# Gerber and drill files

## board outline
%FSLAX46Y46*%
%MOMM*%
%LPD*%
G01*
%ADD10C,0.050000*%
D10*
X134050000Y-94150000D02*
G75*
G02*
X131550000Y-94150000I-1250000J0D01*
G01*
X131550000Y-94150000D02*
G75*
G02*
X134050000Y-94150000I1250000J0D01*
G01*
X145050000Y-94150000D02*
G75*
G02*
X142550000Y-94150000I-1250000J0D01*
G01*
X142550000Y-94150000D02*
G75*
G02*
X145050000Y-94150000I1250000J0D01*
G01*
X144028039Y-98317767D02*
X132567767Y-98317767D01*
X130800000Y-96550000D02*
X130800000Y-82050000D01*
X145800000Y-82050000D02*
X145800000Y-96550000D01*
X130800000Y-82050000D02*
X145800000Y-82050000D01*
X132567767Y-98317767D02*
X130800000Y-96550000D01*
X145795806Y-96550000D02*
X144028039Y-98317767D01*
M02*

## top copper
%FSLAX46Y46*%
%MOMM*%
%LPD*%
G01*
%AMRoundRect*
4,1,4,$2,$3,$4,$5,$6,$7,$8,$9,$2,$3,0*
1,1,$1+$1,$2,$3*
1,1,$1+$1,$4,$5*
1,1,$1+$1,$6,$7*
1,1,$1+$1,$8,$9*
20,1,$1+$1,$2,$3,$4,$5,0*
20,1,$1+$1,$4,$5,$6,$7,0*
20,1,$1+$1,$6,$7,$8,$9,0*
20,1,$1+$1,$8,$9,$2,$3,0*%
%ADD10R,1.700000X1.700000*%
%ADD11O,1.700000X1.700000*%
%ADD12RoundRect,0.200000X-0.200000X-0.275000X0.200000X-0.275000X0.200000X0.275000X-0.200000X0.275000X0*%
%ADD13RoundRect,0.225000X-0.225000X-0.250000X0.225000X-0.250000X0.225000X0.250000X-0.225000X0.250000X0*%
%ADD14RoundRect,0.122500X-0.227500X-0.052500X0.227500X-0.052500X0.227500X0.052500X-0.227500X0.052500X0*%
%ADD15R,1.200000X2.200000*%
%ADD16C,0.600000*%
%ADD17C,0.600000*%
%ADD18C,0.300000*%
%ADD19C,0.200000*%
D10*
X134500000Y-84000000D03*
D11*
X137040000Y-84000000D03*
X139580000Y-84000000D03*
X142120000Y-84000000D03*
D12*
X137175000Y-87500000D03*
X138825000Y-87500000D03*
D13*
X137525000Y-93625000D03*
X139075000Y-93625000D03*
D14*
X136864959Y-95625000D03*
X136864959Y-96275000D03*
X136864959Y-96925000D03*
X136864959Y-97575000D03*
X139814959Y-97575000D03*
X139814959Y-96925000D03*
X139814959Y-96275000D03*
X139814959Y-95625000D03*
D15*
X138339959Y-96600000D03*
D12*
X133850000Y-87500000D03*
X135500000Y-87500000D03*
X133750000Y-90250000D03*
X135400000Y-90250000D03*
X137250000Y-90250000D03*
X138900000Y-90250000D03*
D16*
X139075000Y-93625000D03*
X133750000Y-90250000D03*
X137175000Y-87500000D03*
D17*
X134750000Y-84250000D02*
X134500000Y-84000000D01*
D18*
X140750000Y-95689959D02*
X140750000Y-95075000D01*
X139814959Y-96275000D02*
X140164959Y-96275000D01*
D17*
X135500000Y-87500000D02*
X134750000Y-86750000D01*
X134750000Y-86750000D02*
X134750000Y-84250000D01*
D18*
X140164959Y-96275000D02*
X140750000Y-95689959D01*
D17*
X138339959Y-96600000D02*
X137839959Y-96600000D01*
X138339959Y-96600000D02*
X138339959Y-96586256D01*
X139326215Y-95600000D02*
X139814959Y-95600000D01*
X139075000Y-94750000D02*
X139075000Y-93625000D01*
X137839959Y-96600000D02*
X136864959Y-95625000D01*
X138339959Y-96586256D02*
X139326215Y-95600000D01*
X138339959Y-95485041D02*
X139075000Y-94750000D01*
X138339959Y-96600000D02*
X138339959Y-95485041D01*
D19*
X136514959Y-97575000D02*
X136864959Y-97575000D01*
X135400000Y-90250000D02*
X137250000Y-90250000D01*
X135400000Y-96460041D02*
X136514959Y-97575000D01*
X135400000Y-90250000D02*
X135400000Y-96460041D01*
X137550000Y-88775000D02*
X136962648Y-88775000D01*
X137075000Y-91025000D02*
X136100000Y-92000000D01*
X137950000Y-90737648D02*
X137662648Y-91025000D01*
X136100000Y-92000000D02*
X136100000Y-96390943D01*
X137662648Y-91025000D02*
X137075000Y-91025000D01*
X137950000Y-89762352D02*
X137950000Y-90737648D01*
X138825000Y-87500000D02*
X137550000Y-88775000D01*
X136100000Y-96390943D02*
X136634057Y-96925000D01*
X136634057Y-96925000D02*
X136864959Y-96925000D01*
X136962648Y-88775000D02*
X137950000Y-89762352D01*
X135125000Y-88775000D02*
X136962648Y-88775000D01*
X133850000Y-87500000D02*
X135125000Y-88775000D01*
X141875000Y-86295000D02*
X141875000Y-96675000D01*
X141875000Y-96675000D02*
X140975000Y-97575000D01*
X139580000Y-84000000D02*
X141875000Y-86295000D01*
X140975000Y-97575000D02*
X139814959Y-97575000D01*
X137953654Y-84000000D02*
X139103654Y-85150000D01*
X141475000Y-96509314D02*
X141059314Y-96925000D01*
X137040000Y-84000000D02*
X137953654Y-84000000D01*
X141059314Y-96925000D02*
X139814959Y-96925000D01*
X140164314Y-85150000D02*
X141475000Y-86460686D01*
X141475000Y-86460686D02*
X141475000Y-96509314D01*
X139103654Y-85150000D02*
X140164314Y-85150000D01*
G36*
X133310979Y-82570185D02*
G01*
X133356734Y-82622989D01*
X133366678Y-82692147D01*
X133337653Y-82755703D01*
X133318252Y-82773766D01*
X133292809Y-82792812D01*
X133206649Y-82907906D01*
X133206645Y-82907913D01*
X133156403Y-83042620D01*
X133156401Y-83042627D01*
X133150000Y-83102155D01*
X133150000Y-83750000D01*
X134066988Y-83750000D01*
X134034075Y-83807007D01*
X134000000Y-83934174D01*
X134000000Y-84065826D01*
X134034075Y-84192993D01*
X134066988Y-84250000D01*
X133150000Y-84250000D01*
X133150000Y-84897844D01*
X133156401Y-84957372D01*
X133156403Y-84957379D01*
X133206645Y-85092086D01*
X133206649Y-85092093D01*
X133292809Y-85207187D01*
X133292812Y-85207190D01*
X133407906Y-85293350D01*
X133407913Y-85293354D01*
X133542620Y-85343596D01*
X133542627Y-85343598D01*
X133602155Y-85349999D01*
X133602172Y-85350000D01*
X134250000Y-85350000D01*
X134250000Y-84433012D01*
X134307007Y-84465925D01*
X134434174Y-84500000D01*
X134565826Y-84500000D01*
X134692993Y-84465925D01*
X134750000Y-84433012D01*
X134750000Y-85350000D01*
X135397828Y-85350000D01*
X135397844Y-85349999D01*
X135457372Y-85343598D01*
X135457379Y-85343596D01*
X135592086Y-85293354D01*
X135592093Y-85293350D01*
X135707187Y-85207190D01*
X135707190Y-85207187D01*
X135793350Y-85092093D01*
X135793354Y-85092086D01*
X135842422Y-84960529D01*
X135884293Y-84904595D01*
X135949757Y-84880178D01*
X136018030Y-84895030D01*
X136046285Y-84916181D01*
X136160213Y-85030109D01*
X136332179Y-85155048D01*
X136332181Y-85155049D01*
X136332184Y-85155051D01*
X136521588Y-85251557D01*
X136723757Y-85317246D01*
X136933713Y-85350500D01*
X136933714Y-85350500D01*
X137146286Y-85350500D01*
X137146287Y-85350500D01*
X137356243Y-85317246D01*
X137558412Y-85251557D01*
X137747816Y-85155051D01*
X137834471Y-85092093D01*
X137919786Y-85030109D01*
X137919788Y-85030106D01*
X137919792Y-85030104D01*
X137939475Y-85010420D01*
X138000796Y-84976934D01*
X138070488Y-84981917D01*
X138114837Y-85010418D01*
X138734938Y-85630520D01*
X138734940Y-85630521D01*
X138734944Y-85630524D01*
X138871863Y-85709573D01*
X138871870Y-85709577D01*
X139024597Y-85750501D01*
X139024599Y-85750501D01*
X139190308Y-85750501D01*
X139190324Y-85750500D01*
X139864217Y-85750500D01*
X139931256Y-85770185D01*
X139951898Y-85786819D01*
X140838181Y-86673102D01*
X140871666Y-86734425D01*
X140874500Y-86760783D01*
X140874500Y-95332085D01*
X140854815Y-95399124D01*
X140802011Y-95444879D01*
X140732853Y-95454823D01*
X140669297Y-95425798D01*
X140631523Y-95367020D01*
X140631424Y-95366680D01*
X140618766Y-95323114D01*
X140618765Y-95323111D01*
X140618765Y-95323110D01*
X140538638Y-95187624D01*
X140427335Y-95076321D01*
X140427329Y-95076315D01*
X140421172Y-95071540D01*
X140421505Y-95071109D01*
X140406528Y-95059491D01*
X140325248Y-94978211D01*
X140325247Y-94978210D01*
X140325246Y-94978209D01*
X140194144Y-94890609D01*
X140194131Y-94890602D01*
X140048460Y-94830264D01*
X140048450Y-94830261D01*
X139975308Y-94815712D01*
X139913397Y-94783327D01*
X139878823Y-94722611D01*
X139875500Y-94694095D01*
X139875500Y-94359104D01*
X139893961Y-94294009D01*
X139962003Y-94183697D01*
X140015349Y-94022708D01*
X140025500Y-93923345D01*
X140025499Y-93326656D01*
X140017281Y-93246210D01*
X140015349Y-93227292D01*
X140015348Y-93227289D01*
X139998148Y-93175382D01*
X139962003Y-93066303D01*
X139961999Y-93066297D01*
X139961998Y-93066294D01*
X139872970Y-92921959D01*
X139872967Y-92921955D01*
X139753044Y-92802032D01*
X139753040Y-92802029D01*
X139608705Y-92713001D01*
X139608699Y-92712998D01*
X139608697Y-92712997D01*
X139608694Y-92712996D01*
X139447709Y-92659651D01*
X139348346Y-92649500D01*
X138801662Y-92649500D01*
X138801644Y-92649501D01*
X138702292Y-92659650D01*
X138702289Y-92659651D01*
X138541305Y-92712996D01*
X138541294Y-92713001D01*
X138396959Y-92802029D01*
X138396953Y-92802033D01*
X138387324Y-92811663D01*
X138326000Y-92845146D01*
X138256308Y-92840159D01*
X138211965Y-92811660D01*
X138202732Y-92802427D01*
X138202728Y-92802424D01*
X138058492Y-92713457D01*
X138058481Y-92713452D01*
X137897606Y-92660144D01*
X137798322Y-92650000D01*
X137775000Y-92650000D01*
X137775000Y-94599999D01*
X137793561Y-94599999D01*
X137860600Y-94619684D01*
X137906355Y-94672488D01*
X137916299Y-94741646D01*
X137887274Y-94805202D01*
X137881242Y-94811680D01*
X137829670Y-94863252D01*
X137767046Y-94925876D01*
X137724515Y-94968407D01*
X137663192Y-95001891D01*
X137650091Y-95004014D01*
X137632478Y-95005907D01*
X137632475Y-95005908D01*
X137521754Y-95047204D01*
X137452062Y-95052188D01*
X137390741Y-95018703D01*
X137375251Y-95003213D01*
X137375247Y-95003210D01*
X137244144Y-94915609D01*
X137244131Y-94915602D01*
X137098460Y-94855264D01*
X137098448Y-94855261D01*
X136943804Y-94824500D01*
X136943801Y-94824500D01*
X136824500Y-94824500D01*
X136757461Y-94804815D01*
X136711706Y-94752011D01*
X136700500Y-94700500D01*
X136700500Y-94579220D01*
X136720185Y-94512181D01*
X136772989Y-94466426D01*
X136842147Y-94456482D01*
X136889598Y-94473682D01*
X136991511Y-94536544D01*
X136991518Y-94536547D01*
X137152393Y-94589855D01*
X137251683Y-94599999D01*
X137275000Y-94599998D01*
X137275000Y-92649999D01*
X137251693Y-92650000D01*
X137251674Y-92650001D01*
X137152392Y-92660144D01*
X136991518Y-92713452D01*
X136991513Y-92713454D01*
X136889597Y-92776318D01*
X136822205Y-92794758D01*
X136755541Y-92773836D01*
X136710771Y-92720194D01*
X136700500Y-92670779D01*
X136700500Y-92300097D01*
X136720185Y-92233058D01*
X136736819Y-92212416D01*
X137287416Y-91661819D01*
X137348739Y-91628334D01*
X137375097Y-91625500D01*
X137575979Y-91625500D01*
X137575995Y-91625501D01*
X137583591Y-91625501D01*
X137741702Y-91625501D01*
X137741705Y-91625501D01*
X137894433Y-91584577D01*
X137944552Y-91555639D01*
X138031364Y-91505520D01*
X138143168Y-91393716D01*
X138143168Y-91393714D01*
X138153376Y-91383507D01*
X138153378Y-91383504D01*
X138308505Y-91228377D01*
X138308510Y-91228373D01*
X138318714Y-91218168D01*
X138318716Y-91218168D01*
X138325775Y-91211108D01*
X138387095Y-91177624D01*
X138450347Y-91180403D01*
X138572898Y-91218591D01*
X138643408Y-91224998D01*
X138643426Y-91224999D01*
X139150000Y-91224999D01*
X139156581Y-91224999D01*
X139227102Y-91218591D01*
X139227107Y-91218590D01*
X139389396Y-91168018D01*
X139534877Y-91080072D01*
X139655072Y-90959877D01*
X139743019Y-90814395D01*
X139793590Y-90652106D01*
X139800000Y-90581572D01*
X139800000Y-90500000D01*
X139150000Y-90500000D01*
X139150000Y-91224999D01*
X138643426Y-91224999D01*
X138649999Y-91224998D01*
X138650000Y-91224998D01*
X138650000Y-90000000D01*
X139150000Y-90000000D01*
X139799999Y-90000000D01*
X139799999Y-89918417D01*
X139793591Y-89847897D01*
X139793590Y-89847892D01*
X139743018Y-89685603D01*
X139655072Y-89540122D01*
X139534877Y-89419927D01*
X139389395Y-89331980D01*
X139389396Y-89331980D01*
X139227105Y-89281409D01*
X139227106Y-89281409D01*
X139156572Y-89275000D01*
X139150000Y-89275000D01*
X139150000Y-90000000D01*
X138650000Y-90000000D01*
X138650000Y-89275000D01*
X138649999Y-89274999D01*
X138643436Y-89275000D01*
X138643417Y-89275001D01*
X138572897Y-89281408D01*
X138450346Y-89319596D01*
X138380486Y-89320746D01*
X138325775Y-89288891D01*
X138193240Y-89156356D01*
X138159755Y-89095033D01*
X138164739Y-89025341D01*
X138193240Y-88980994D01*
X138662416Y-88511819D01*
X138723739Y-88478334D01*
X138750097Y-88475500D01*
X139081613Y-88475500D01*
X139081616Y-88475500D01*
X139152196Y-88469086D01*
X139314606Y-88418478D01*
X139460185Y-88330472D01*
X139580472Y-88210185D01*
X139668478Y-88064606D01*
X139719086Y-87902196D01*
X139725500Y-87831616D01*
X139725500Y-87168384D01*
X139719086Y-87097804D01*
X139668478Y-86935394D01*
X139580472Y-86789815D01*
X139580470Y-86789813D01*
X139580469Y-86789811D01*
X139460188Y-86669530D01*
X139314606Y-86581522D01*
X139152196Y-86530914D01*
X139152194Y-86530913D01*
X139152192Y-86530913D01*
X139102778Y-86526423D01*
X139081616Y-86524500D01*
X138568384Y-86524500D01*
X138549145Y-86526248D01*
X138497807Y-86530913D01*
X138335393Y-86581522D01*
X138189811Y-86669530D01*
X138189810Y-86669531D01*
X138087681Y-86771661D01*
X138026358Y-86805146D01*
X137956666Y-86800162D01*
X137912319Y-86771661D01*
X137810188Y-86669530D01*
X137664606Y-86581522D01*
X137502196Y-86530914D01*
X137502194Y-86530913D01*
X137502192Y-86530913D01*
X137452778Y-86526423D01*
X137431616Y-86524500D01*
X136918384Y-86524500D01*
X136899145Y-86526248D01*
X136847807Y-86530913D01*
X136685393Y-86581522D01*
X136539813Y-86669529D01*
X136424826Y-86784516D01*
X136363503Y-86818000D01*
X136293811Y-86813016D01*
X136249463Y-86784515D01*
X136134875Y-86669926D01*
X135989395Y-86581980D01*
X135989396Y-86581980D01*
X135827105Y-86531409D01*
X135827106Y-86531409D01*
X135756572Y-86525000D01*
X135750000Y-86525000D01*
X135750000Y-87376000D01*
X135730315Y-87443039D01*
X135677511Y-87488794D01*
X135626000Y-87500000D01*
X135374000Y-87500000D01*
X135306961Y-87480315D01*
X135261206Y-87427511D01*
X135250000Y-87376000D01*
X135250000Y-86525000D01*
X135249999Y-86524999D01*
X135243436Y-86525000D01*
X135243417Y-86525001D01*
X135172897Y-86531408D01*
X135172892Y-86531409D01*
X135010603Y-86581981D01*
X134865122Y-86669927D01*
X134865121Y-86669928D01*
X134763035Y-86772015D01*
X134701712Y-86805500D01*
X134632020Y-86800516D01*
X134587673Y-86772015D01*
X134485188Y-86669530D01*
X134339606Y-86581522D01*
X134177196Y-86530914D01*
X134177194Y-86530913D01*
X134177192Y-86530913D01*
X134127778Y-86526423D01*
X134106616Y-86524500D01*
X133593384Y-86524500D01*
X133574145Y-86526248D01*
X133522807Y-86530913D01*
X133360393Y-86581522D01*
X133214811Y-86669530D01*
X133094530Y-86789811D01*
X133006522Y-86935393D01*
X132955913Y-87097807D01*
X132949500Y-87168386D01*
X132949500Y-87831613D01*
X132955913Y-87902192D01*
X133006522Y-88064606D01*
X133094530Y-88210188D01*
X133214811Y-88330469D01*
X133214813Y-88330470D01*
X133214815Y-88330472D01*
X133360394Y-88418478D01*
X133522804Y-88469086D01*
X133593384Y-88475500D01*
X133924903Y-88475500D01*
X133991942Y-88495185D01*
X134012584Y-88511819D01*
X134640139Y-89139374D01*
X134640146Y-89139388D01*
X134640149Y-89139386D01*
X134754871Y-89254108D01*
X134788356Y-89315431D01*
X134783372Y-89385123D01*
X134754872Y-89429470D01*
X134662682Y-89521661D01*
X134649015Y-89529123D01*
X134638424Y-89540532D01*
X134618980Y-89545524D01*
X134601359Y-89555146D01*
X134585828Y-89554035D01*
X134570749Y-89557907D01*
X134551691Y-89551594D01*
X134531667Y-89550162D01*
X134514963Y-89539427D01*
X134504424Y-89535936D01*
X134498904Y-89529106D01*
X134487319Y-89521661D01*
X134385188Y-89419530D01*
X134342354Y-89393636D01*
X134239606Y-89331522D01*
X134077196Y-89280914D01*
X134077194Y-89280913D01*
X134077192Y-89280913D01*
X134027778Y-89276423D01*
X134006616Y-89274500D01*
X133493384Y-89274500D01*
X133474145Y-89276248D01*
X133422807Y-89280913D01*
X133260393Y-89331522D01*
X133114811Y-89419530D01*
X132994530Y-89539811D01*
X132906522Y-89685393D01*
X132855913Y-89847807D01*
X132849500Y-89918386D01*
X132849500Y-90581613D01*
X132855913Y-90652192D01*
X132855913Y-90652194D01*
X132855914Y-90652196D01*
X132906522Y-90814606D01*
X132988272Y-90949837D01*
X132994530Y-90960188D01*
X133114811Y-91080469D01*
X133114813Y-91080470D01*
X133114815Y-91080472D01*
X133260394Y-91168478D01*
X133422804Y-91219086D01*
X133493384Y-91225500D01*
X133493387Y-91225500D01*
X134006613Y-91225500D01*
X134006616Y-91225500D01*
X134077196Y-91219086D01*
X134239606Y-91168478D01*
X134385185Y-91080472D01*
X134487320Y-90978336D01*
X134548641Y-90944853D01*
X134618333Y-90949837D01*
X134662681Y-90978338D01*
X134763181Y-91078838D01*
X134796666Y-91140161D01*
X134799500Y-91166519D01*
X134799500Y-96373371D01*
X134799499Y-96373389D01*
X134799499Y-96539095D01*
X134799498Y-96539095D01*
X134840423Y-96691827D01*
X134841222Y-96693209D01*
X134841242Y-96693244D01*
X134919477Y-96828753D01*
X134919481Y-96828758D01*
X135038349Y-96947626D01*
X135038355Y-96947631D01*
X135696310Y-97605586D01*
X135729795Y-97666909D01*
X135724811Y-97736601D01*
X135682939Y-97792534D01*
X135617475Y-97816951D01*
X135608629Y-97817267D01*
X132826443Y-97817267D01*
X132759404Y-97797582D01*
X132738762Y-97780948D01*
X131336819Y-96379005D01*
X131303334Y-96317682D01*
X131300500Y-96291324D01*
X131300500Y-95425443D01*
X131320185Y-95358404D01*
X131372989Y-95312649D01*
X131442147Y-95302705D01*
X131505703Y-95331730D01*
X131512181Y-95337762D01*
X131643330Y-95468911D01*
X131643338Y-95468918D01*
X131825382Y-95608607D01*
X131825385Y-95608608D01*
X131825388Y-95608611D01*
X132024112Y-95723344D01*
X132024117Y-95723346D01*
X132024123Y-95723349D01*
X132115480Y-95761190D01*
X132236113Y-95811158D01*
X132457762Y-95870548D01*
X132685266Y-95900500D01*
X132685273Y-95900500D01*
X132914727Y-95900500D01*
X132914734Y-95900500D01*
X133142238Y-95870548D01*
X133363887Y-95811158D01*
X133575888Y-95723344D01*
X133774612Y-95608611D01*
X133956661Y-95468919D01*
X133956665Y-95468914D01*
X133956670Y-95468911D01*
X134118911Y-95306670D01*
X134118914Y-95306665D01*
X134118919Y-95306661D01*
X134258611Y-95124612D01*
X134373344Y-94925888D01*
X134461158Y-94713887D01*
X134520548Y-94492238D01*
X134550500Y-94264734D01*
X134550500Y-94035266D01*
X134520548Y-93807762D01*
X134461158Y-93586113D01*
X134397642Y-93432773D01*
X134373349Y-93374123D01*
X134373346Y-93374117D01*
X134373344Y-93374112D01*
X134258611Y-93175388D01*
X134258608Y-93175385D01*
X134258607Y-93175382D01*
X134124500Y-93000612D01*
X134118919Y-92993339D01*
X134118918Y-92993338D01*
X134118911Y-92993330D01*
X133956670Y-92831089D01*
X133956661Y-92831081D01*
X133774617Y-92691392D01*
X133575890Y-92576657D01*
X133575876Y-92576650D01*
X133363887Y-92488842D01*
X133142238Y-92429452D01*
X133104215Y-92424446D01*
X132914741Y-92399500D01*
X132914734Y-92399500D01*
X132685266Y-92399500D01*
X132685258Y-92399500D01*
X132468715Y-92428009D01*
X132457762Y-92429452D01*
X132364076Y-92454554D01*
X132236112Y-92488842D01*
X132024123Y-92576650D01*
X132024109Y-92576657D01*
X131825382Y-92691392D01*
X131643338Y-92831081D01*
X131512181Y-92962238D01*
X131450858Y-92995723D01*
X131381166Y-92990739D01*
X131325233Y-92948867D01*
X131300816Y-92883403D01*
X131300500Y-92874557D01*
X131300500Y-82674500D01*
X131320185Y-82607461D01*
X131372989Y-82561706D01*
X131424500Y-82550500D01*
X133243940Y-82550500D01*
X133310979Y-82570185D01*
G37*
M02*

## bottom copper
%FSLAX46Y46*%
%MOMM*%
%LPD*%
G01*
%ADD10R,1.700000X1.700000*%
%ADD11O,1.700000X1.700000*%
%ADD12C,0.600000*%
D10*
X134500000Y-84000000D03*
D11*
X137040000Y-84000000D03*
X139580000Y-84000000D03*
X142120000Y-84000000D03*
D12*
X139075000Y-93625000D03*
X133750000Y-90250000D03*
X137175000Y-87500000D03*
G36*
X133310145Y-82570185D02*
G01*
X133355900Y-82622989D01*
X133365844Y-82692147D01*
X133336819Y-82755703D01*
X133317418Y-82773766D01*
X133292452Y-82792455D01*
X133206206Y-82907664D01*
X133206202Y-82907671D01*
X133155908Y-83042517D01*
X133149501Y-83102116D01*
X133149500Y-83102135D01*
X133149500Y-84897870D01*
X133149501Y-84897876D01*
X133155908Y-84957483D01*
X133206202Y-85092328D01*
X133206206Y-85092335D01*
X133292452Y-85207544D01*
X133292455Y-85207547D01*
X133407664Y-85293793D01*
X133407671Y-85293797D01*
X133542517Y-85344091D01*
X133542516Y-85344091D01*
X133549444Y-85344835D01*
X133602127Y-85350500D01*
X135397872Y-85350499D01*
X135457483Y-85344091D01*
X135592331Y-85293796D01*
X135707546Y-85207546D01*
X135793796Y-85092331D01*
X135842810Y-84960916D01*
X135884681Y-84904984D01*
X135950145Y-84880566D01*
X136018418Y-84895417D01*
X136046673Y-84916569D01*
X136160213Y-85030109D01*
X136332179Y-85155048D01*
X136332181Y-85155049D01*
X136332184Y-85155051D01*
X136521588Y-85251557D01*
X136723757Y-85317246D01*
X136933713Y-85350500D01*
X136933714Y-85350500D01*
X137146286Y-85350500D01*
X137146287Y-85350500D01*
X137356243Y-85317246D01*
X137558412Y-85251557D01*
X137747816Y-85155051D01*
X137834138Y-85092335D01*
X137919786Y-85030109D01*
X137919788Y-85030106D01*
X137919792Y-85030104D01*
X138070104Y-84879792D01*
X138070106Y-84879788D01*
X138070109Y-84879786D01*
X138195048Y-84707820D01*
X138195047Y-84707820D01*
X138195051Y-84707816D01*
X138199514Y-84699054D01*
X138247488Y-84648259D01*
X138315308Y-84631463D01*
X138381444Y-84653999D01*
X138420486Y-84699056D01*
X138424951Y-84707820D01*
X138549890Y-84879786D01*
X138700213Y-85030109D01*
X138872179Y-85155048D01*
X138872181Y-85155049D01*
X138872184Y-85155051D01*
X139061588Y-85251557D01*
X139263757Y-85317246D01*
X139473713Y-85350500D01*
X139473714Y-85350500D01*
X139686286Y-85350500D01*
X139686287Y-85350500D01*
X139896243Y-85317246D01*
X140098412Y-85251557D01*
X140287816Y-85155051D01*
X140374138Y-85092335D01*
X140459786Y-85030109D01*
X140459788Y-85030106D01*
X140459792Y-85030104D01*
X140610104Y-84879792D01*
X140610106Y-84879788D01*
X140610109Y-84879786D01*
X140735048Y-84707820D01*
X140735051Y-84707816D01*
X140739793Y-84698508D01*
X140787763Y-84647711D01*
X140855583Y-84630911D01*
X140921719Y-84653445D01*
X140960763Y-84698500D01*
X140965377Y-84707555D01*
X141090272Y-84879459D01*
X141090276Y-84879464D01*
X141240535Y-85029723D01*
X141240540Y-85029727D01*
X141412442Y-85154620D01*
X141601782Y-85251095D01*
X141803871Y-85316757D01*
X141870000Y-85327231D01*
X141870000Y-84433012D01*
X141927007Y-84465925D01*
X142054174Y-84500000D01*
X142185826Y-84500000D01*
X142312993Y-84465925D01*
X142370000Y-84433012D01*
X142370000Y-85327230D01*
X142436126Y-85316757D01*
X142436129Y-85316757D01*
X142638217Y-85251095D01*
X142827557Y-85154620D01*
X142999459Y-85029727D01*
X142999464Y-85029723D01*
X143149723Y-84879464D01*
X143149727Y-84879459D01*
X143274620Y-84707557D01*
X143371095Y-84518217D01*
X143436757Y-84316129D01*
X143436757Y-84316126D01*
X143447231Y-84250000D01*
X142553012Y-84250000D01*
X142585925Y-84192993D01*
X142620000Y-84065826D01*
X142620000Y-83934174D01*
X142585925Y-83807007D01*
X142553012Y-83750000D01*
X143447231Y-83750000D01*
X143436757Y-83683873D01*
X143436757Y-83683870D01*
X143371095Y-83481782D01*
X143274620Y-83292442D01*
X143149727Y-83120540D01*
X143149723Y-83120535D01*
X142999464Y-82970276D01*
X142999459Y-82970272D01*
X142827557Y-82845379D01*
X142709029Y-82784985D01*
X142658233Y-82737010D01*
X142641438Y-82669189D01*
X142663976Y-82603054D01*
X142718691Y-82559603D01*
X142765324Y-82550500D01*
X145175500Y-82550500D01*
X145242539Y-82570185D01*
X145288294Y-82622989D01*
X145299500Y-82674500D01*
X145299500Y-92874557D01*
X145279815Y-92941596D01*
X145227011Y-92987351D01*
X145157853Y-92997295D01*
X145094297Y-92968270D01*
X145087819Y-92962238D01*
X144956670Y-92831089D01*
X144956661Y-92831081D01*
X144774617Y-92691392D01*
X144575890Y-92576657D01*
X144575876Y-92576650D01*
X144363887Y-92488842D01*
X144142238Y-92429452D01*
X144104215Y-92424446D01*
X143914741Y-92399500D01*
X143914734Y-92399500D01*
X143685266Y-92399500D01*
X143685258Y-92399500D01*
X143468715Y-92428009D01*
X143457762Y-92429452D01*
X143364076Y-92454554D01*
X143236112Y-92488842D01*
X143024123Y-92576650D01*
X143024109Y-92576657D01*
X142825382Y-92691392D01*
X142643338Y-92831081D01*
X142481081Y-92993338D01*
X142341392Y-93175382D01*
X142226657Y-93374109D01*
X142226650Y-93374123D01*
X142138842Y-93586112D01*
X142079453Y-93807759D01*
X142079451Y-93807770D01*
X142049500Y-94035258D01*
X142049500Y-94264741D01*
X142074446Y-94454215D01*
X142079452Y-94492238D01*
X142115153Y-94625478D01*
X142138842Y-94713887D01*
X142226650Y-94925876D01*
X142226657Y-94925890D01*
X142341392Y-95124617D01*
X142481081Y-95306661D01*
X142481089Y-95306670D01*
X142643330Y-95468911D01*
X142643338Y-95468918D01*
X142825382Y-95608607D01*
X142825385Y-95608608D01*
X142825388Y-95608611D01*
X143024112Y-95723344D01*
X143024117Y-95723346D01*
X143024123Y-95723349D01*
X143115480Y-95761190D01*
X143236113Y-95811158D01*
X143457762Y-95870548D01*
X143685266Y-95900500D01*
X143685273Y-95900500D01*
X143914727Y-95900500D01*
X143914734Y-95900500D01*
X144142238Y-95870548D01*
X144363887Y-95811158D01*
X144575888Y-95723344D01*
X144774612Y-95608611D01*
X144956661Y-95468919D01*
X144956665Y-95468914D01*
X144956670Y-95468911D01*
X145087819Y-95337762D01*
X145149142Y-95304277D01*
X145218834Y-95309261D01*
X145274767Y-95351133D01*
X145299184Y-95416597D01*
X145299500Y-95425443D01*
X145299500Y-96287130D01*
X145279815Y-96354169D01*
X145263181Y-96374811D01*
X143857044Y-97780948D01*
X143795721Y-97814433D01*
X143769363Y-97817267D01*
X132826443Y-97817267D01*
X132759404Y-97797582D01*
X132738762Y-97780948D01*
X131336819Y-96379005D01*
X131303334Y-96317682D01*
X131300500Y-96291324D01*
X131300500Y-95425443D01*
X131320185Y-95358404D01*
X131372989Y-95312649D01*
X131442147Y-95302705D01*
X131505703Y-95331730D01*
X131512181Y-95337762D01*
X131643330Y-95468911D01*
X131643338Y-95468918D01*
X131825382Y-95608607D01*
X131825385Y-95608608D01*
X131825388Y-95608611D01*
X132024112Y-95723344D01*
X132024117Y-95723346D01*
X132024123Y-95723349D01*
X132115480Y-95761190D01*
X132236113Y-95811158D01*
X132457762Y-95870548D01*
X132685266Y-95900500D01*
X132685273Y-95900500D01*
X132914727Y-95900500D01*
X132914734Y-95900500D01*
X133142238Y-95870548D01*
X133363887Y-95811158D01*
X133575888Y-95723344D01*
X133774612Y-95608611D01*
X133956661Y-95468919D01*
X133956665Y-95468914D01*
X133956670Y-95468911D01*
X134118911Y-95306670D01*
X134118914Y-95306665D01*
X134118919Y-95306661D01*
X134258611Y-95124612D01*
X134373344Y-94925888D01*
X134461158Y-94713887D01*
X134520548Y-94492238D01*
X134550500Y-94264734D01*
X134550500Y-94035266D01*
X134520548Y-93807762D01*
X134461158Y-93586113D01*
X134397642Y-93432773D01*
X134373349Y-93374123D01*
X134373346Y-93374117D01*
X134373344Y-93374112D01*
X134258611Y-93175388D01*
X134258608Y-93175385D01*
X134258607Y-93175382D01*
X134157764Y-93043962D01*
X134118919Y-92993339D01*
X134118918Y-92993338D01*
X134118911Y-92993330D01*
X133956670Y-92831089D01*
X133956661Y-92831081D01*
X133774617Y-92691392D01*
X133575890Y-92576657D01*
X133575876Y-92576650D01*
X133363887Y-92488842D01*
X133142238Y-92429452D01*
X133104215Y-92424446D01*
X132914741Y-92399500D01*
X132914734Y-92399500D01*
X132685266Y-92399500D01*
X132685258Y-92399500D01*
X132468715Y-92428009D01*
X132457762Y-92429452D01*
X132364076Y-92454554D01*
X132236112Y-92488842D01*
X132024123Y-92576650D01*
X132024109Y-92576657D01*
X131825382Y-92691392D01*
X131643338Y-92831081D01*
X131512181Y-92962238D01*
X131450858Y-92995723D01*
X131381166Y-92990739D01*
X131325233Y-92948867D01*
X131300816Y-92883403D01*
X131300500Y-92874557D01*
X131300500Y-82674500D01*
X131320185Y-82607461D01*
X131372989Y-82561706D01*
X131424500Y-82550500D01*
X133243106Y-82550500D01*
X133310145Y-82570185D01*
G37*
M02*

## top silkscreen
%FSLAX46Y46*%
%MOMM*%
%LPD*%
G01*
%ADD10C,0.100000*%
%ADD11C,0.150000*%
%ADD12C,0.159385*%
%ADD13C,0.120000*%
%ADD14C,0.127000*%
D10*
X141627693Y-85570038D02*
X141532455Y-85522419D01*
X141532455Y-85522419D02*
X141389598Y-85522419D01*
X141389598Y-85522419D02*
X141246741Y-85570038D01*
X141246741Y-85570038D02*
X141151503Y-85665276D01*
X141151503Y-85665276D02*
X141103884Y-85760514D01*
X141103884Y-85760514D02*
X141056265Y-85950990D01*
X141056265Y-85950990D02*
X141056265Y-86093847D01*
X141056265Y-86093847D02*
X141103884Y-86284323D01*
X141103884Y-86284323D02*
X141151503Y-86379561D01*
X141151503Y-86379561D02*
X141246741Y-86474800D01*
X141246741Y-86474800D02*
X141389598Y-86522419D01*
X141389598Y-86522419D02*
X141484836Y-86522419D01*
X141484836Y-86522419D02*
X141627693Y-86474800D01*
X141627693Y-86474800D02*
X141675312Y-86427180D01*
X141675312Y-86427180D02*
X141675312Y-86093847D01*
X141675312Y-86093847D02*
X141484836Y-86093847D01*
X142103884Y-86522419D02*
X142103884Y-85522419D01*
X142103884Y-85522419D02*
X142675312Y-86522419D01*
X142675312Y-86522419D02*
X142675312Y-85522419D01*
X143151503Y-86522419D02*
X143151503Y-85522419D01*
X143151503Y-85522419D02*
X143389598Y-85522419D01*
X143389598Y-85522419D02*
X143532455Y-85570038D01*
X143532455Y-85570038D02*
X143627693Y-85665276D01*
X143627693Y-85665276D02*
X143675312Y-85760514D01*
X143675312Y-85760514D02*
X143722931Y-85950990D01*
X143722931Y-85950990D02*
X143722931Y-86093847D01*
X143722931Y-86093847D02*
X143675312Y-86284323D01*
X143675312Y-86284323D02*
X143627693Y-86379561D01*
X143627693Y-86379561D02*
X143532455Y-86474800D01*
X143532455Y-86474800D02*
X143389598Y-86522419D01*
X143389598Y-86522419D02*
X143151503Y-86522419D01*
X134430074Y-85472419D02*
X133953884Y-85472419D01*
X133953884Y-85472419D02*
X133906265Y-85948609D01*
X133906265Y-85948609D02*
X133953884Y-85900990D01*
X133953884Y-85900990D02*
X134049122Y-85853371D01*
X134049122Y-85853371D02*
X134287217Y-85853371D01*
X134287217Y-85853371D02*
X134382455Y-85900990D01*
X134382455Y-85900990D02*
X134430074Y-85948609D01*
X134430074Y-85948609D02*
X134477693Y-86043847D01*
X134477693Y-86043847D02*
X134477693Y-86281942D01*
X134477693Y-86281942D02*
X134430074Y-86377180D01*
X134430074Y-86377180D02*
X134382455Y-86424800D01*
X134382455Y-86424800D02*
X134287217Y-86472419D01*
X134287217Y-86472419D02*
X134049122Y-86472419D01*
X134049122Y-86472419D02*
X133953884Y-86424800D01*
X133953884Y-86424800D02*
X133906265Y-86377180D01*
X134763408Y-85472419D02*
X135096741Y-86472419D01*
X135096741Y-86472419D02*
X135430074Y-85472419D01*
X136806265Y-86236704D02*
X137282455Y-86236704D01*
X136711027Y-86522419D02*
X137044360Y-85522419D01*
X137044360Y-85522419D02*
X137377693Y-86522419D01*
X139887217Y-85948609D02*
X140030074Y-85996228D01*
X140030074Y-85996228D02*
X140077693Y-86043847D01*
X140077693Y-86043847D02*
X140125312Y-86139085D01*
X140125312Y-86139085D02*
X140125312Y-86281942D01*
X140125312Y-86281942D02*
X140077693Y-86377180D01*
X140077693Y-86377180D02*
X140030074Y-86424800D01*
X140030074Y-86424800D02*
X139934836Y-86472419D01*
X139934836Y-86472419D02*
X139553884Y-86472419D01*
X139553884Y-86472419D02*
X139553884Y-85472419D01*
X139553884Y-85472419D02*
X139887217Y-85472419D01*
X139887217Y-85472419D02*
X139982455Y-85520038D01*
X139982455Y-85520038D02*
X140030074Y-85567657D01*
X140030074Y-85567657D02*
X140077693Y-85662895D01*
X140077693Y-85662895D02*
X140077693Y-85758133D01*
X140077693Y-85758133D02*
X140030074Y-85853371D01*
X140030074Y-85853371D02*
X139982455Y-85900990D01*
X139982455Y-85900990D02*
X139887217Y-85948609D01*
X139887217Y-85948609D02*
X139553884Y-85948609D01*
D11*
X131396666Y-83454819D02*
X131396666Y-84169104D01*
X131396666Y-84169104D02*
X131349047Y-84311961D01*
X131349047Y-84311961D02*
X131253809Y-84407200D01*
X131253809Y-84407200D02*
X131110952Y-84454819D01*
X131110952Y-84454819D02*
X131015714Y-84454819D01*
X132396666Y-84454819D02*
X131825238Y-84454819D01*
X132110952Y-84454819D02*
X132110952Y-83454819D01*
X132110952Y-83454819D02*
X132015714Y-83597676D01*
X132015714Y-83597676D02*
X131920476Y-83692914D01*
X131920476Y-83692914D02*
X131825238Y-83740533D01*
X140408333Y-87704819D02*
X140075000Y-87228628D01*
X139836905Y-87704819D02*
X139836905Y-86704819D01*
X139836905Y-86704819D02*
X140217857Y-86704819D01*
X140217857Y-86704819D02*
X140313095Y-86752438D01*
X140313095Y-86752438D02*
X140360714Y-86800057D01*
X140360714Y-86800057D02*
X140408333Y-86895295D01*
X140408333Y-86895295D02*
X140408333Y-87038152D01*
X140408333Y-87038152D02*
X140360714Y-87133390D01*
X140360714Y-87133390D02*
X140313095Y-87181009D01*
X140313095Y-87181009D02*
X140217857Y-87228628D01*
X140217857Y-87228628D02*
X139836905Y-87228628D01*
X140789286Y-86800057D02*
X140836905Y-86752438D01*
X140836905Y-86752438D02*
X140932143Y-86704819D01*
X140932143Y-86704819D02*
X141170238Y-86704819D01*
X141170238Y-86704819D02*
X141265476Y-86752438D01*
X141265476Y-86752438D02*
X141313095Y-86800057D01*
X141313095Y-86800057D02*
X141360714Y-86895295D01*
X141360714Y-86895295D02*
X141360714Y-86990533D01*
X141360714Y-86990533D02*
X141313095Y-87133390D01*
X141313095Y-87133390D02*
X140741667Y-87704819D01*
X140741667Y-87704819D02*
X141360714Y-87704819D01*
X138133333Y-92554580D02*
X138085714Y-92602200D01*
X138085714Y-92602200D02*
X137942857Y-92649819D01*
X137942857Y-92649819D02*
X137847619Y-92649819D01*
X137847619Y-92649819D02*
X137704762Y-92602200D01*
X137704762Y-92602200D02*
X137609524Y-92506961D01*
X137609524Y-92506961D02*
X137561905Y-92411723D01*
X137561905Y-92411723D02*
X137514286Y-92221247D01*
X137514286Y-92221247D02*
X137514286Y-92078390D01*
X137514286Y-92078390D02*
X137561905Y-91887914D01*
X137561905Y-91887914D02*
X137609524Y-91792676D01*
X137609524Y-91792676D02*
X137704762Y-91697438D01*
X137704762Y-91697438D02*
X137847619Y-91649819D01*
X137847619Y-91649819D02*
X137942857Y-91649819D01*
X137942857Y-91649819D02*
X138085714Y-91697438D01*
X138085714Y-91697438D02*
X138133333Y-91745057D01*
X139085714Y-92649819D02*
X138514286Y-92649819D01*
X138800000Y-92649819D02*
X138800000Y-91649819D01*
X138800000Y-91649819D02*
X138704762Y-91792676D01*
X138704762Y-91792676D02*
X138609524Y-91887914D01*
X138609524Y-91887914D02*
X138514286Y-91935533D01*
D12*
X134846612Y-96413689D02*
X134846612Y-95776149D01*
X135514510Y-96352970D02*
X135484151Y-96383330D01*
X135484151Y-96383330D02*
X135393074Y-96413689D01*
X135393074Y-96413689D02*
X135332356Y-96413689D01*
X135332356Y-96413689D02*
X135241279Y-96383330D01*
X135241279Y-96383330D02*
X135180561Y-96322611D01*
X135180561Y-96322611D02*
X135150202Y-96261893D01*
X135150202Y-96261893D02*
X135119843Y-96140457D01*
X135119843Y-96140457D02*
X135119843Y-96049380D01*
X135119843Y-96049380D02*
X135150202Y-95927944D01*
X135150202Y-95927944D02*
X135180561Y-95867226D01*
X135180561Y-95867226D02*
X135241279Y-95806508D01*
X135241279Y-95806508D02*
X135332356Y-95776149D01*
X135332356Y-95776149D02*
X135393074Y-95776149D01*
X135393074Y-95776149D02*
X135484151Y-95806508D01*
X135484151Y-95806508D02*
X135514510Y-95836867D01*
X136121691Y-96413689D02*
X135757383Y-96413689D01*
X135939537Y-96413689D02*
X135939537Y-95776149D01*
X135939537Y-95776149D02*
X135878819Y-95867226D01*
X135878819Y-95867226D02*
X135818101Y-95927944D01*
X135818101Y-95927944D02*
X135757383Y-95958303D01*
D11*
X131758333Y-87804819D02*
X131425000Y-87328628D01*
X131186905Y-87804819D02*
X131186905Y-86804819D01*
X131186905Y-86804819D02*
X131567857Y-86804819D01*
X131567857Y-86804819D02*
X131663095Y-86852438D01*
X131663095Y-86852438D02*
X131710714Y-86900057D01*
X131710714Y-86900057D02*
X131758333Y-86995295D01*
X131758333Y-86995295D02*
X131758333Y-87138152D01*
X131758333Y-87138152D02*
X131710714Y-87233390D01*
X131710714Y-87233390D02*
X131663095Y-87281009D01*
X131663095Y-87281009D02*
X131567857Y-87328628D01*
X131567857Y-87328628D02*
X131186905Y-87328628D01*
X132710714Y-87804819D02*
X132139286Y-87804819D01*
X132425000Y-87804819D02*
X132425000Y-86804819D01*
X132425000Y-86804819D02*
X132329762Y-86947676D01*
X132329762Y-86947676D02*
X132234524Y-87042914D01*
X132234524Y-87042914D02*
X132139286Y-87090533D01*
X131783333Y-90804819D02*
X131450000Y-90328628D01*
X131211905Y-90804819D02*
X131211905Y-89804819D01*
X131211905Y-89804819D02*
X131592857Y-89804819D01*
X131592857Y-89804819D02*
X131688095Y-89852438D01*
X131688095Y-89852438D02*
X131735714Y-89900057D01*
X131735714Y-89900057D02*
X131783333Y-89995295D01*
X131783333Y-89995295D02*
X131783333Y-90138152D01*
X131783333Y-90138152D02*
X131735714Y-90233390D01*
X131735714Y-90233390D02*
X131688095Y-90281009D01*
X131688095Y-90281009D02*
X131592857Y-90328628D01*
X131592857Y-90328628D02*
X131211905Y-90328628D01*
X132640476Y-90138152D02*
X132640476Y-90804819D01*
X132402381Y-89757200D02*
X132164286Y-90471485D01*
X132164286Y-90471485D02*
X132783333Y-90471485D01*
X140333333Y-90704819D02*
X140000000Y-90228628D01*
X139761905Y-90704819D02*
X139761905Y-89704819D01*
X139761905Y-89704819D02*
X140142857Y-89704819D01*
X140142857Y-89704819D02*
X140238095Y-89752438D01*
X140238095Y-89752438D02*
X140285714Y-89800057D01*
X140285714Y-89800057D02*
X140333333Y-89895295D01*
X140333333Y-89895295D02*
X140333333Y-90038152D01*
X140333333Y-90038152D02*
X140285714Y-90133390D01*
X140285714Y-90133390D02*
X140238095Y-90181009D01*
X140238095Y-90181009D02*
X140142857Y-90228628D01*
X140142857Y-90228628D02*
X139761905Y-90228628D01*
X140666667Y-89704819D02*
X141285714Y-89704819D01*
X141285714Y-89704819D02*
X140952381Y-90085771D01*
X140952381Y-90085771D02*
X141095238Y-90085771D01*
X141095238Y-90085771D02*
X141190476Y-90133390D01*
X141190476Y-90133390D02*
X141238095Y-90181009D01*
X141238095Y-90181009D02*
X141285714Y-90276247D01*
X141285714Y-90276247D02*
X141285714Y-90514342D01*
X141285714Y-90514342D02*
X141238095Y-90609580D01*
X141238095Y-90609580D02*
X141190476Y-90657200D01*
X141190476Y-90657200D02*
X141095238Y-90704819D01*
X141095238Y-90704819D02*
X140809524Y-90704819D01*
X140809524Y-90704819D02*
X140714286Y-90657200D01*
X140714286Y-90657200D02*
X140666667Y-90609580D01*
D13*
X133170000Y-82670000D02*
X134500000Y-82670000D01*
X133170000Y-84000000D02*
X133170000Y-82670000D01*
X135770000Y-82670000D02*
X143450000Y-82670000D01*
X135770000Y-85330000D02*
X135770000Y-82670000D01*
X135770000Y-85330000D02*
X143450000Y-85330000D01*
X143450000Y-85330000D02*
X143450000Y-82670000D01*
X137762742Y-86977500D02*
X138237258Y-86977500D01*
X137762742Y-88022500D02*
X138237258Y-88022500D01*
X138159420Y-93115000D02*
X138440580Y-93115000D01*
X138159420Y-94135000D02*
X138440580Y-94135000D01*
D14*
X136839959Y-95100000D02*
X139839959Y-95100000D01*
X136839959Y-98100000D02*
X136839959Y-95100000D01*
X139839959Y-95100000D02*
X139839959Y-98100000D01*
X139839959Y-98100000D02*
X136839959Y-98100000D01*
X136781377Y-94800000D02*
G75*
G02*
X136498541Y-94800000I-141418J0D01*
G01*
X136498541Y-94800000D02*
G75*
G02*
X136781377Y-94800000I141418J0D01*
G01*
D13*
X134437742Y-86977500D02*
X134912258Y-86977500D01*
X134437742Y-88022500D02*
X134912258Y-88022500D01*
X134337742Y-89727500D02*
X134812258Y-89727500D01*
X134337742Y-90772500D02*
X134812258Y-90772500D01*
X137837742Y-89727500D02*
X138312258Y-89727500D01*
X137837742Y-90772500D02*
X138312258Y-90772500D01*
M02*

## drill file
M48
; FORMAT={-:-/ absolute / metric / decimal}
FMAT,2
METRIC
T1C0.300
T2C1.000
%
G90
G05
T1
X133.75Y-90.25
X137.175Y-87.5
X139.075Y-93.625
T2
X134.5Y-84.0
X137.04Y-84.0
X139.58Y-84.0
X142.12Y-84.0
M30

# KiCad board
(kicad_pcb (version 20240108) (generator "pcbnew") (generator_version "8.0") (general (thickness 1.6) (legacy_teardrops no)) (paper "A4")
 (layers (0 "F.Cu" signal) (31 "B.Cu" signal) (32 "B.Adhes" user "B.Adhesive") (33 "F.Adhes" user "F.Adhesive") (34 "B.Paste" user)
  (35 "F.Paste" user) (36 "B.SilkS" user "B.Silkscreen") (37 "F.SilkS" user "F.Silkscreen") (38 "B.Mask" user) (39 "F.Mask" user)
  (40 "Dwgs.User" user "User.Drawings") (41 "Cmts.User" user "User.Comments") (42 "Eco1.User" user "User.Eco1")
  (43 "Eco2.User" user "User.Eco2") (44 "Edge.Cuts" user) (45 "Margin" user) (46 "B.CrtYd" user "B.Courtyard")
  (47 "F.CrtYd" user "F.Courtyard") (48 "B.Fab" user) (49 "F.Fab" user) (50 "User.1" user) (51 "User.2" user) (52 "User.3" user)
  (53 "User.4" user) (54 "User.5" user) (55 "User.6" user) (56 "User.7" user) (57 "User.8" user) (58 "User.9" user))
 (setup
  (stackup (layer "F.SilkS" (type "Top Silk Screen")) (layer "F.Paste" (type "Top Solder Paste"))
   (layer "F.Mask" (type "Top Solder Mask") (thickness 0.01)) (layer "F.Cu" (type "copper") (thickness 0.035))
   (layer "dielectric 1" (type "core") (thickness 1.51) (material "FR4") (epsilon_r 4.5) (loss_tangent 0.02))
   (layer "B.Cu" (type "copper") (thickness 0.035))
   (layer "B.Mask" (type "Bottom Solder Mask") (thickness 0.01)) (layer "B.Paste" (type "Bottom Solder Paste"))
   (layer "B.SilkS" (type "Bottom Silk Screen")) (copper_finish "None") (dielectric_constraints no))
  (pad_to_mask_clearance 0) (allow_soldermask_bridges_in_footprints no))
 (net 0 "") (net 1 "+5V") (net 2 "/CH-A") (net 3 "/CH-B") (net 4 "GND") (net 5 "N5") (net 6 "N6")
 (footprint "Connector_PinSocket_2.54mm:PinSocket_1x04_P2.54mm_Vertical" (layer "F.Cu") (at 134.5 84 90)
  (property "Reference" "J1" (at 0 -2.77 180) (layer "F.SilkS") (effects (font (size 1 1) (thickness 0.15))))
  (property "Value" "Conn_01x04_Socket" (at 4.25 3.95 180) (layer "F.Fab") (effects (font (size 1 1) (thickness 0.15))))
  (fp_line (start 1.33 -1.33) (end 1.33 0) (stroke (width 0.12) (type solid)) (layer "F.SilkS"))
  (fp_line (start 0 -1.33) (end 1.33 -1.33) (stroke (width 0.12) (type solid)) (layer "F.SilkS"))
  (fp_line (start 1.33 1.27) (end 1.33 8.95) (stroke (width 0.12) (type solid)) (layer "F.SilkS"))
  (fp_line (start -1.33 1.27) (end 1.33 1.27) (stroke (width 0.12) (type solid)) (layer "F.SilkS"))
  (fp_line (start -1.33 1.27) (end -1.33 8.95) (stroke (width 0.12) (type solid)) (layer "F.SilkS"))
  (fp_line (start -1.33 8.95) (end 1.33 8.95) (stroke (width 0.12) (type solid)) (layer "F.SilkS"))
  (pad "1" thru_hole rect (at 0 0 90) (size 1.7 1.7) (drill 1) (layers "*.Cu" "*.Mask") (remove_unused_layers no) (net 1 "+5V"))
  (pad "2" thru_hole oval (at 0 2.54 90) (size 1.7 1.7) (drill 1) (layers "*.Cu" "*.Mask") (remove_unused_layers no) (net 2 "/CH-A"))
  (pad "3" thru_hole oval (at 0 5.08 90) (size 1.7 1.7) (drill 1) (layers "*.Cu" "*.Mask") (remove_unused_layers no) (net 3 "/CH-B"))
  (pad "4" thru_hole oval (at 0 7.62 90) (size 1.7 1.7) (drill 1) (layers "*.Cu" "*.Mask") (remove_unused_layers no) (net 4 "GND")))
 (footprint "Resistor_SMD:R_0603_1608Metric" (layer "F.Cu") (at 138 87.5)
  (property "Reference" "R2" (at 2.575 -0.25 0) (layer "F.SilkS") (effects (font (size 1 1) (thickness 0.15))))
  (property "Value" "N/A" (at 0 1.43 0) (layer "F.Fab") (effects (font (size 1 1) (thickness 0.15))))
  (fp_line (start -0.237258 -0.5225) (end 0.237258 -0.5225) (stroke (width 0.12) (type solid)) (layer "F.SilkS"))
  (fp_line (start -0.237258 0.5225) (end 0.237258 0.5225) (stroke (width 0.12) (type solid)) (layer "F.SilkS"))
  (pad "1" smd roundrect (at -0.825 0) (size 0.8 0.95) (layers "F.Cu" "F.Paste" "F.Mask") (roundrect_rratio 0.25) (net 4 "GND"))
  (pad "2" smd roundrect (at 0.825 0) (size 0.8 0.95) (layers "F.Cu" "F.Paste" "F.Mask") (roundrect_rratio 0.25) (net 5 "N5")))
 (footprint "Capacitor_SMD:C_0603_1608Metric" (layer "F.Cu") (at 138.3 93.625)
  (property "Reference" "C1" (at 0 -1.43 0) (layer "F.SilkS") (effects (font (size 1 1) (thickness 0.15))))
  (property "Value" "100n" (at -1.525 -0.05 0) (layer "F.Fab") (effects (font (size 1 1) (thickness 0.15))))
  (fp_line (start -0.14058 -0.51) (end 0.14058 -0.51) (stroke (width 0.12) (type solid)) (layer "F.SilkS"))
  (fp_line (start -0.14058 0.51) (end 0.14058 0.51) (stroke (width 0.12) (type solid)) (layer "F.SilkS"))
  (pad "1" smd roundrect (at -0.775 0) (size 0.9 0.95) (layers "F.Cu" "F.Paste" "F.Mask") (roundrect_rratio 0.25) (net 1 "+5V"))
  (pad "2" smd roundrect (at 0.775 0) (size 0.9 0.95) (layers "F.Cu" "F.Paste" "F.Mask") (roundrect_rratio 0.25) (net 4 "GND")))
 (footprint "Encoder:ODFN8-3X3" (layer "F.Cu") (at 138.339959 96.6)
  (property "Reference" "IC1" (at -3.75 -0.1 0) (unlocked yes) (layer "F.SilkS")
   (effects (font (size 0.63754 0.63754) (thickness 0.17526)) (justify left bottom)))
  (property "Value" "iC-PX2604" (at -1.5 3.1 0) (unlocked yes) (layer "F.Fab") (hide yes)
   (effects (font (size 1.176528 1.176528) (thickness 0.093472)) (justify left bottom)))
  (fp_line (start -1.5 -1.5) (end 1.5 -1.5) (stroke (width 0.127) (type solid)) (layer "F.SilkS"))
  (fp_line (start -1.5 1.5) (end -1.5 -1.5) (stroke (width 0.127) (type solid)) (layer "F.SilkS"))
  (fp_line (start 1.5 -1.5) (end 1.5 1.5) (stroke (width 0.127) (type solid)) (layer "F.SilkS"))
  (fp_line (start 1.5 1.5) (end -1.5 1.5) (stroke (width 0.127) (type solid)) (layer "F.SilkS"))
  (fp_circle (center -1.7 -1.8) (end -1.558582 -1.8) (stroke (width 0.127) (type solid)) (fill none) (layer "F.SilkS"))
  (pad "1" smd roundrect (at -1.475 -0.975) (size 0.7 0.35) (layers "F.Cu" "F.Paste" "F.Mask") (roundrect_rratio 0.35) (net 4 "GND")
   (solder_mask_margin 0.075) (thermal_bridge_angle 0))
  (pad "2" smd roundrect (at -1.475 -0.325) (size 0.7 0.35) (layers "F.Cu" "F.Paste" "F.Mask") (roundrect_rratio 0.35) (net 4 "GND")
   (solder_mask_margin 0.075) (thermal_bridge_angle 0))
  (pad "3" smd roundrect (at -1.475 0.325) (size 0.7 0.35) (layers "F.Cu" "F.Paste" "F.Mask") (roundrect_rratio 0.35) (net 5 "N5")
   (solder_mask_margin 0.075) (thermal_bridge_angle 0))
  (pad "4" smd roundrect (at -1.475 0.975) (size 0.7 0.35) (layers "F.Cu" "F.Paste" "F.Mask") (roundrect_rratio 0.35) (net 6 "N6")
   (solder_mask_margin 0.075) (thermal_bridge_angle 0))
  (pad "5" smd roundrect (at 1.475 0.975) (size 0.7 0.35) (layers "F.Cu" "F.Paste" "F.Mask") (roundrect_rratio 0.35) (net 3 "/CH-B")
   (solder_mask_margin 0.075) (thermal_bridge_angle 0))
  (pad "6" smd roundrect (at 1.475 0.325) (size 0.7 0.35) (layers "F.Cu" "F.Paste" "F.Mask") (roundrect_rratio 0.35) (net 2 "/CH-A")
   (solder_mask_margin 0.075) (thermal_bridge_angle 0))
  (pad "7" smd roundrect (at 1.475 -0.325) (size 0.7 0.35) (layers "F.Cu" "F.Paste" "F.Mask") (roundrect_rratio 0.35) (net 1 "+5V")
   (solder_mask_margin 0.075) (thermal_bridge_angle 0))
  (pad "8" smd roundrect (at 1.475 -0.975) (size 0.7 0.35) (layers "F.Cu" "F.Paste" "F.Mask") (roundrect_rratio 0.35) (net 4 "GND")
   (solder_mask_margin 0.075) (thermal_bridge_angle 0))
  (pad "BP" smd rect (at 0 0) (size 1.2 2.2) (layers "F.Cu" "F.Mask") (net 4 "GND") (solder_mask_margin 0.075) (thermal_bridge_angle 0)))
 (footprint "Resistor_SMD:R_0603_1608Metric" (layer "F.Cu") (at 134.675 87.5)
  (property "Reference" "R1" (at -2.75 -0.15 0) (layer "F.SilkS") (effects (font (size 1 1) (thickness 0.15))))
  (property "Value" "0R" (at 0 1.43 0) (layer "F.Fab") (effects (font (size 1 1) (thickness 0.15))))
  (fp_line (start -0.237258 -0.5225) (end 0.237258 -0.5225) (stroke (width 0.12) (type solid)) (layer "F.SilkS"))
  (fp_line (start -0.237258 0.5225) (end 0.237258 0.5225) (stroke (width 0.12) (type solid)) (layer "F.SilkS"))
  (pad "1" smd roundrect (at -0.825 0) (size 0.8 0.95) (layers "F.Cu" "F.Paste" "F.Mask") (roundrect_rratio 0.25) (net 5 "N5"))
  (pad "2" smd roundrect (at 0.825 0) (size 0.8 0.95) (layers "F.Cu" "F.Paste" "F.Mask") (roundrect_rratio 0.25) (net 1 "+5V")))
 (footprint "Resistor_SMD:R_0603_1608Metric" (layer "F.Cu") (at 134.575 90.25)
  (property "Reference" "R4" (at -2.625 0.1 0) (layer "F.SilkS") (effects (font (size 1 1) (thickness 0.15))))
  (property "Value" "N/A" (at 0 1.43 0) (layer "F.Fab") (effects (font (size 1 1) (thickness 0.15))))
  (fp_line (start -0.237258 -0.5225) (end 0.237258 -0.5225) (stroke (width 0.12) (type solid)) (layer "F.SilkS"))
  (fp_line (start -0.237258 0.5225) (end 0.237258 0.5225) (stroke (width 0.12) (type solid)) (layer "F.SilkS"))
  (pad "1" smd roundrect (at -0.825 0) (size 0.8 0.95) (layers "F.Cu" "F.Paste" "F.Mask") (roundrect_rratio 0.25) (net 4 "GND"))
  (pad "2" smd roundrect (at 0.825 0) (size 0.8 0.95) (layers "F.Cu" "F.Paste" "F.Mask") (roundrect_rratio 0.25) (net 6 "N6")))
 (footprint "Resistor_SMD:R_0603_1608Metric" (layer "F.Cu") (at 138.075 90.25)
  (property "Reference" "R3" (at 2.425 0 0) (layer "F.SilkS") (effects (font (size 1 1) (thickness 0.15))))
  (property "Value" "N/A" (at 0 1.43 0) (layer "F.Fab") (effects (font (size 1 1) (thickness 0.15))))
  (fp_line (start -0.237258 -0.5225) (end 0.237258 -0.5225) (stroke (width 0.12) (type solid)) (layer "F.SilkS"))
  (fp_line (start -0.237258 0.5225) (end 0.237258 0.5225) (stroke (width 0.12) (type solid)) (layer "F.SilkS"))
  (pad "1" smd roundrect (at -0.825 0) (size 0.8 0.95) (layers "F.Cu" "F.Paste" "F.Mask") (roundrect_rratio 0.25) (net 6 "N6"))
  (pad "2" smd roundrect (at 0.825 0) (size 0.8 0.95) (layers "F.Cu" "F.Paste" "F.Mask") (roundrect_rratio 0.25) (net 1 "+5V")))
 (gr_circle (center 132.8 94.15) (end 134.05 94.15) (stroke (width 0.05) (type default)) (fill none) (layer "Edge.Cuts"))
 (gr_circle (center 143.8 94.15) (end 145.05 94.15) (stroke (width 0.05) (type default)) (fill none) (layer "Edge.Cuts"))
 (gr_line (start 144.028039 98.317767) (end 132.567767 98.317767) (stroke (width 0.05) (type default)) (layer "Edge.Cuts"))
 (gr_line (start 130.8 96.55) (end 130.8 82.05) (stroke (width 0.05) (type default)) (layer "Edge.Cuts"))
 (gr_line (start 145.8 82.05) (end 145.8 96.55) (stroke (width 0.05) (type default)) (layer "Edge.Cuts"))
 (gr_line (start 130.8 82.05) (end 145.8 82.05) (stroke (width 0.05) (type default)) (layer "Edge.Cuts"))
 (gr_line (start 132.567767 98.317767) (end 130.8 96.55) (stroke (width 0.05) (type default)) (layer "Edge.Cuts"))
 (gr_line (start 145.795806 96.55) (end 144.028039 98.317767) (stroke (width 0.05) (type default)) (layer "Edge.Cuts"))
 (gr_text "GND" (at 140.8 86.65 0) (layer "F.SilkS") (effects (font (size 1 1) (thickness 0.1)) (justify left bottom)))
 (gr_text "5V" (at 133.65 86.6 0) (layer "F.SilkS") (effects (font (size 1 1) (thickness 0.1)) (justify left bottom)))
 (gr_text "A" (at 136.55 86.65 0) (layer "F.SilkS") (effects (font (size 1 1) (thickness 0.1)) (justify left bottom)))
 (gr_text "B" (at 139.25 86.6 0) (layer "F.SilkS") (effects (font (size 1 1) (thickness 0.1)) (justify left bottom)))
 (segment (start 134.75 84.25) (end 134.5 84) (width 0.6) (layer "F.Cu") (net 1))
 (segment (start 140.75 95.689959) (end 140.75 95.075) (width 0.3) (layer "F.Cu") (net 1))
 (segment (start 139.814959 96.275) (end 140.164959 96.275) (width 0.3) (layer "F.Cu") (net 1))
 (segment (start 135.5 87.5) (end 134.75 86.75) (width 0.6) (layer "F.Cu") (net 1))
 (segment (start 134.75 86.75) (end 134.75 84.25) (width 0.6) (layer "F.Cu") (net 1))
 (segment (start 140.164959 96.275) (end 140.75 95.689959) (width 0.3) (layer "F.Cu") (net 1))
 (segment (start 138.339959 96.6) (end 137.839959 96.6) (width 0.6) (layer "F.Cu") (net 4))
 (segment (start 138.339959 96.6) (end 138.339959 96.586256) (width 0.6) (layer "F.Cu") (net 4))
 (segment (start 139.326215 95.6) (end 139.814959 95.6) (width 0.6) (layer "F.Cu") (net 4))
 (segment (start 139.075 94.75) (end 139.075 93.625) (width 0.6) (layer "F.Cu") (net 4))
 (segment (start 137.839959 96.6) (end 136.864959 95.625) (width 0.6) (layer "F.Cu") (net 4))
 (segment (start 138.339959 96.586256) (end 139.326215 95.6) (width 0.6) (layer "F.Cu") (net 4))
 (segment (start 138.339959 95.485041) (end 139.075 94.75) (width 0.6) (layer "F.Cu") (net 4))
 (segment (start 138.339959 96.6) (end 138.339959 95.485041) (width 0.6) (layer "F.Cu") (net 4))
 (via (at 139.075 93.625) (size 0.6) (drill 0.3) (layers "F.Cu" "B.Cu") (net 4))
 (via (at 133.75 90.25) (size 0.6) (drill 0.3) (layers "F.Cu" "B.Cu") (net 4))
 (via (at 137.175 87.5) (size 0.6) (drill 0.3) (layers "F.Cu" "B.Cu") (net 4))
 (segment (start 136.514959 97.575) (end 136.864959 97.575) (width 0.2) (layer "F.Cu") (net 6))
 (segment (start 135.4 90.25) (end 137.25 90.25) (width 0.2) (layer "F.Cu") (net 6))
 (segment (start 135.4 96.460041) (end 136.514959 97.575) (width 0.2) (layer "F.Cu") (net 6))
 (segment (start 135.4 90.25) (end 135.4 96.460041) (width 0.2) (layer "F.Cu") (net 6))
 (segment (start 137.55 88.775) (end 136.962648 88.775) (width 0.2) (layer "F.Cu") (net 5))
 (segment (start 137.075 91.025) (end 136.1 92) (width 0.2) (layer "F.Cu") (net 5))
 (segment (start 137.95 90.737648) (end 137.662648 91.025) (width 0.2) (layer "F.Cu") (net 5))
 (segment (start 136.1 92) (end 136.1 96.390943) (width 0.2) (layer "F.Cu") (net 5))
 (segment (start 137.662648 91.025) (end 137.075 91.025) (width 0.2) (layer "F.Cu") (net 5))
 (segment (start 137.95 89.762352) (end 137.95 90.737648) (width 0.2) (layer "F.Cu") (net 5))
 (segment (start 138.825 87.5) (end 137.55 88.775) (width 0.2) (layer "F.Cu") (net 5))
 (segment (start 136.1 96.390943) (end 136.634057 96.925) (width 0.2) (layer "F.Cu") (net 5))
 (segment (start 136.634057 96.925) (end 136.864959 96.925) (width 0.2) (layer "F.Cu") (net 5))
 (segment (start 136.962648 88.775) (end 137.95 89.762352) (width 0.2) (layer "F.Cu") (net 5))
 (segment (start 135.125 88.775) (end 136.962648 88.775) (width 0.2) (layer "F.Cu") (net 5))
 (segment (start 133.85 87.5) (end 135.125 88.775) (width 0.2) (layer "F.Cu") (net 5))
 (segment (start 141.875 86.295) (end 141.875 96.675) (width 0.2) (layer "F.Cu") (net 3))
 (segment (start 141.875 96.675) (end 140.975 97.575) (width 0.2) (layer "F.Cu") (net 3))
 (segment (start 139.58 84) (end 141.875 86.295) (width 0.2) (layer "F.Cu") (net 3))
 (segment (start 140.975 97.575) (end 139.814959 97.575) (width 0.2) (layer "F.Cu") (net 3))
 (segment (start 137.953654 84) (end 139.103654 85.15) (width 0.2) (layer "F.Cu") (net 2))
 (segment (start 141.475 96.509314) (end 141.059314 96.925) (width 0.2) (layer "F.Cu") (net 2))
 (segment (start 137.04 84) (end 137.953654 84) (width 0.2) (layer "F.Cu") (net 2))
 (segment (start 141.059314 96.925) (end 139.814959 96.925) (width 0.2) (layer "F.Cu") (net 2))
 (segment (start 140.164314 85.15) (end 141.475 86.460686) (width 0.2) (layer "F.Cu") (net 2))
 (segment (start 141.475 86.460686) (end 141.475 96.509314) (width 0.2) (layer "F.Cu") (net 2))
 (segment (start 139.103654 85.15) (end 140.164314 85.15) (width 0.2) (layer "F.Cu") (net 2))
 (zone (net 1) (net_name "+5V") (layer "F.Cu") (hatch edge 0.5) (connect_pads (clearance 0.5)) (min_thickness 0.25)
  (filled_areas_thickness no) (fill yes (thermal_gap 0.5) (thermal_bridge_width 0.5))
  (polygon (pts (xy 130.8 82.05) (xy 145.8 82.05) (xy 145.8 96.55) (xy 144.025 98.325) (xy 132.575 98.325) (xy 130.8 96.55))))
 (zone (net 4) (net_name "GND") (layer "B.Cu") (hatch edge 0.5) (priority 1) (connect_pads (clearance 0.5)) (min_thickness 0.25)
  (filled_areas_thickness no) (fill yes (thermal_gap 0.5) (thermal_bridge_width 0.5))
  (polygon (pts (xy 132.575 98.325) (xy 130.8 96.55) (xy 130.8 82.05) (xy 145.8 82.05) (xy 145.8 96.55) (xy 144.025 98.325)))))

